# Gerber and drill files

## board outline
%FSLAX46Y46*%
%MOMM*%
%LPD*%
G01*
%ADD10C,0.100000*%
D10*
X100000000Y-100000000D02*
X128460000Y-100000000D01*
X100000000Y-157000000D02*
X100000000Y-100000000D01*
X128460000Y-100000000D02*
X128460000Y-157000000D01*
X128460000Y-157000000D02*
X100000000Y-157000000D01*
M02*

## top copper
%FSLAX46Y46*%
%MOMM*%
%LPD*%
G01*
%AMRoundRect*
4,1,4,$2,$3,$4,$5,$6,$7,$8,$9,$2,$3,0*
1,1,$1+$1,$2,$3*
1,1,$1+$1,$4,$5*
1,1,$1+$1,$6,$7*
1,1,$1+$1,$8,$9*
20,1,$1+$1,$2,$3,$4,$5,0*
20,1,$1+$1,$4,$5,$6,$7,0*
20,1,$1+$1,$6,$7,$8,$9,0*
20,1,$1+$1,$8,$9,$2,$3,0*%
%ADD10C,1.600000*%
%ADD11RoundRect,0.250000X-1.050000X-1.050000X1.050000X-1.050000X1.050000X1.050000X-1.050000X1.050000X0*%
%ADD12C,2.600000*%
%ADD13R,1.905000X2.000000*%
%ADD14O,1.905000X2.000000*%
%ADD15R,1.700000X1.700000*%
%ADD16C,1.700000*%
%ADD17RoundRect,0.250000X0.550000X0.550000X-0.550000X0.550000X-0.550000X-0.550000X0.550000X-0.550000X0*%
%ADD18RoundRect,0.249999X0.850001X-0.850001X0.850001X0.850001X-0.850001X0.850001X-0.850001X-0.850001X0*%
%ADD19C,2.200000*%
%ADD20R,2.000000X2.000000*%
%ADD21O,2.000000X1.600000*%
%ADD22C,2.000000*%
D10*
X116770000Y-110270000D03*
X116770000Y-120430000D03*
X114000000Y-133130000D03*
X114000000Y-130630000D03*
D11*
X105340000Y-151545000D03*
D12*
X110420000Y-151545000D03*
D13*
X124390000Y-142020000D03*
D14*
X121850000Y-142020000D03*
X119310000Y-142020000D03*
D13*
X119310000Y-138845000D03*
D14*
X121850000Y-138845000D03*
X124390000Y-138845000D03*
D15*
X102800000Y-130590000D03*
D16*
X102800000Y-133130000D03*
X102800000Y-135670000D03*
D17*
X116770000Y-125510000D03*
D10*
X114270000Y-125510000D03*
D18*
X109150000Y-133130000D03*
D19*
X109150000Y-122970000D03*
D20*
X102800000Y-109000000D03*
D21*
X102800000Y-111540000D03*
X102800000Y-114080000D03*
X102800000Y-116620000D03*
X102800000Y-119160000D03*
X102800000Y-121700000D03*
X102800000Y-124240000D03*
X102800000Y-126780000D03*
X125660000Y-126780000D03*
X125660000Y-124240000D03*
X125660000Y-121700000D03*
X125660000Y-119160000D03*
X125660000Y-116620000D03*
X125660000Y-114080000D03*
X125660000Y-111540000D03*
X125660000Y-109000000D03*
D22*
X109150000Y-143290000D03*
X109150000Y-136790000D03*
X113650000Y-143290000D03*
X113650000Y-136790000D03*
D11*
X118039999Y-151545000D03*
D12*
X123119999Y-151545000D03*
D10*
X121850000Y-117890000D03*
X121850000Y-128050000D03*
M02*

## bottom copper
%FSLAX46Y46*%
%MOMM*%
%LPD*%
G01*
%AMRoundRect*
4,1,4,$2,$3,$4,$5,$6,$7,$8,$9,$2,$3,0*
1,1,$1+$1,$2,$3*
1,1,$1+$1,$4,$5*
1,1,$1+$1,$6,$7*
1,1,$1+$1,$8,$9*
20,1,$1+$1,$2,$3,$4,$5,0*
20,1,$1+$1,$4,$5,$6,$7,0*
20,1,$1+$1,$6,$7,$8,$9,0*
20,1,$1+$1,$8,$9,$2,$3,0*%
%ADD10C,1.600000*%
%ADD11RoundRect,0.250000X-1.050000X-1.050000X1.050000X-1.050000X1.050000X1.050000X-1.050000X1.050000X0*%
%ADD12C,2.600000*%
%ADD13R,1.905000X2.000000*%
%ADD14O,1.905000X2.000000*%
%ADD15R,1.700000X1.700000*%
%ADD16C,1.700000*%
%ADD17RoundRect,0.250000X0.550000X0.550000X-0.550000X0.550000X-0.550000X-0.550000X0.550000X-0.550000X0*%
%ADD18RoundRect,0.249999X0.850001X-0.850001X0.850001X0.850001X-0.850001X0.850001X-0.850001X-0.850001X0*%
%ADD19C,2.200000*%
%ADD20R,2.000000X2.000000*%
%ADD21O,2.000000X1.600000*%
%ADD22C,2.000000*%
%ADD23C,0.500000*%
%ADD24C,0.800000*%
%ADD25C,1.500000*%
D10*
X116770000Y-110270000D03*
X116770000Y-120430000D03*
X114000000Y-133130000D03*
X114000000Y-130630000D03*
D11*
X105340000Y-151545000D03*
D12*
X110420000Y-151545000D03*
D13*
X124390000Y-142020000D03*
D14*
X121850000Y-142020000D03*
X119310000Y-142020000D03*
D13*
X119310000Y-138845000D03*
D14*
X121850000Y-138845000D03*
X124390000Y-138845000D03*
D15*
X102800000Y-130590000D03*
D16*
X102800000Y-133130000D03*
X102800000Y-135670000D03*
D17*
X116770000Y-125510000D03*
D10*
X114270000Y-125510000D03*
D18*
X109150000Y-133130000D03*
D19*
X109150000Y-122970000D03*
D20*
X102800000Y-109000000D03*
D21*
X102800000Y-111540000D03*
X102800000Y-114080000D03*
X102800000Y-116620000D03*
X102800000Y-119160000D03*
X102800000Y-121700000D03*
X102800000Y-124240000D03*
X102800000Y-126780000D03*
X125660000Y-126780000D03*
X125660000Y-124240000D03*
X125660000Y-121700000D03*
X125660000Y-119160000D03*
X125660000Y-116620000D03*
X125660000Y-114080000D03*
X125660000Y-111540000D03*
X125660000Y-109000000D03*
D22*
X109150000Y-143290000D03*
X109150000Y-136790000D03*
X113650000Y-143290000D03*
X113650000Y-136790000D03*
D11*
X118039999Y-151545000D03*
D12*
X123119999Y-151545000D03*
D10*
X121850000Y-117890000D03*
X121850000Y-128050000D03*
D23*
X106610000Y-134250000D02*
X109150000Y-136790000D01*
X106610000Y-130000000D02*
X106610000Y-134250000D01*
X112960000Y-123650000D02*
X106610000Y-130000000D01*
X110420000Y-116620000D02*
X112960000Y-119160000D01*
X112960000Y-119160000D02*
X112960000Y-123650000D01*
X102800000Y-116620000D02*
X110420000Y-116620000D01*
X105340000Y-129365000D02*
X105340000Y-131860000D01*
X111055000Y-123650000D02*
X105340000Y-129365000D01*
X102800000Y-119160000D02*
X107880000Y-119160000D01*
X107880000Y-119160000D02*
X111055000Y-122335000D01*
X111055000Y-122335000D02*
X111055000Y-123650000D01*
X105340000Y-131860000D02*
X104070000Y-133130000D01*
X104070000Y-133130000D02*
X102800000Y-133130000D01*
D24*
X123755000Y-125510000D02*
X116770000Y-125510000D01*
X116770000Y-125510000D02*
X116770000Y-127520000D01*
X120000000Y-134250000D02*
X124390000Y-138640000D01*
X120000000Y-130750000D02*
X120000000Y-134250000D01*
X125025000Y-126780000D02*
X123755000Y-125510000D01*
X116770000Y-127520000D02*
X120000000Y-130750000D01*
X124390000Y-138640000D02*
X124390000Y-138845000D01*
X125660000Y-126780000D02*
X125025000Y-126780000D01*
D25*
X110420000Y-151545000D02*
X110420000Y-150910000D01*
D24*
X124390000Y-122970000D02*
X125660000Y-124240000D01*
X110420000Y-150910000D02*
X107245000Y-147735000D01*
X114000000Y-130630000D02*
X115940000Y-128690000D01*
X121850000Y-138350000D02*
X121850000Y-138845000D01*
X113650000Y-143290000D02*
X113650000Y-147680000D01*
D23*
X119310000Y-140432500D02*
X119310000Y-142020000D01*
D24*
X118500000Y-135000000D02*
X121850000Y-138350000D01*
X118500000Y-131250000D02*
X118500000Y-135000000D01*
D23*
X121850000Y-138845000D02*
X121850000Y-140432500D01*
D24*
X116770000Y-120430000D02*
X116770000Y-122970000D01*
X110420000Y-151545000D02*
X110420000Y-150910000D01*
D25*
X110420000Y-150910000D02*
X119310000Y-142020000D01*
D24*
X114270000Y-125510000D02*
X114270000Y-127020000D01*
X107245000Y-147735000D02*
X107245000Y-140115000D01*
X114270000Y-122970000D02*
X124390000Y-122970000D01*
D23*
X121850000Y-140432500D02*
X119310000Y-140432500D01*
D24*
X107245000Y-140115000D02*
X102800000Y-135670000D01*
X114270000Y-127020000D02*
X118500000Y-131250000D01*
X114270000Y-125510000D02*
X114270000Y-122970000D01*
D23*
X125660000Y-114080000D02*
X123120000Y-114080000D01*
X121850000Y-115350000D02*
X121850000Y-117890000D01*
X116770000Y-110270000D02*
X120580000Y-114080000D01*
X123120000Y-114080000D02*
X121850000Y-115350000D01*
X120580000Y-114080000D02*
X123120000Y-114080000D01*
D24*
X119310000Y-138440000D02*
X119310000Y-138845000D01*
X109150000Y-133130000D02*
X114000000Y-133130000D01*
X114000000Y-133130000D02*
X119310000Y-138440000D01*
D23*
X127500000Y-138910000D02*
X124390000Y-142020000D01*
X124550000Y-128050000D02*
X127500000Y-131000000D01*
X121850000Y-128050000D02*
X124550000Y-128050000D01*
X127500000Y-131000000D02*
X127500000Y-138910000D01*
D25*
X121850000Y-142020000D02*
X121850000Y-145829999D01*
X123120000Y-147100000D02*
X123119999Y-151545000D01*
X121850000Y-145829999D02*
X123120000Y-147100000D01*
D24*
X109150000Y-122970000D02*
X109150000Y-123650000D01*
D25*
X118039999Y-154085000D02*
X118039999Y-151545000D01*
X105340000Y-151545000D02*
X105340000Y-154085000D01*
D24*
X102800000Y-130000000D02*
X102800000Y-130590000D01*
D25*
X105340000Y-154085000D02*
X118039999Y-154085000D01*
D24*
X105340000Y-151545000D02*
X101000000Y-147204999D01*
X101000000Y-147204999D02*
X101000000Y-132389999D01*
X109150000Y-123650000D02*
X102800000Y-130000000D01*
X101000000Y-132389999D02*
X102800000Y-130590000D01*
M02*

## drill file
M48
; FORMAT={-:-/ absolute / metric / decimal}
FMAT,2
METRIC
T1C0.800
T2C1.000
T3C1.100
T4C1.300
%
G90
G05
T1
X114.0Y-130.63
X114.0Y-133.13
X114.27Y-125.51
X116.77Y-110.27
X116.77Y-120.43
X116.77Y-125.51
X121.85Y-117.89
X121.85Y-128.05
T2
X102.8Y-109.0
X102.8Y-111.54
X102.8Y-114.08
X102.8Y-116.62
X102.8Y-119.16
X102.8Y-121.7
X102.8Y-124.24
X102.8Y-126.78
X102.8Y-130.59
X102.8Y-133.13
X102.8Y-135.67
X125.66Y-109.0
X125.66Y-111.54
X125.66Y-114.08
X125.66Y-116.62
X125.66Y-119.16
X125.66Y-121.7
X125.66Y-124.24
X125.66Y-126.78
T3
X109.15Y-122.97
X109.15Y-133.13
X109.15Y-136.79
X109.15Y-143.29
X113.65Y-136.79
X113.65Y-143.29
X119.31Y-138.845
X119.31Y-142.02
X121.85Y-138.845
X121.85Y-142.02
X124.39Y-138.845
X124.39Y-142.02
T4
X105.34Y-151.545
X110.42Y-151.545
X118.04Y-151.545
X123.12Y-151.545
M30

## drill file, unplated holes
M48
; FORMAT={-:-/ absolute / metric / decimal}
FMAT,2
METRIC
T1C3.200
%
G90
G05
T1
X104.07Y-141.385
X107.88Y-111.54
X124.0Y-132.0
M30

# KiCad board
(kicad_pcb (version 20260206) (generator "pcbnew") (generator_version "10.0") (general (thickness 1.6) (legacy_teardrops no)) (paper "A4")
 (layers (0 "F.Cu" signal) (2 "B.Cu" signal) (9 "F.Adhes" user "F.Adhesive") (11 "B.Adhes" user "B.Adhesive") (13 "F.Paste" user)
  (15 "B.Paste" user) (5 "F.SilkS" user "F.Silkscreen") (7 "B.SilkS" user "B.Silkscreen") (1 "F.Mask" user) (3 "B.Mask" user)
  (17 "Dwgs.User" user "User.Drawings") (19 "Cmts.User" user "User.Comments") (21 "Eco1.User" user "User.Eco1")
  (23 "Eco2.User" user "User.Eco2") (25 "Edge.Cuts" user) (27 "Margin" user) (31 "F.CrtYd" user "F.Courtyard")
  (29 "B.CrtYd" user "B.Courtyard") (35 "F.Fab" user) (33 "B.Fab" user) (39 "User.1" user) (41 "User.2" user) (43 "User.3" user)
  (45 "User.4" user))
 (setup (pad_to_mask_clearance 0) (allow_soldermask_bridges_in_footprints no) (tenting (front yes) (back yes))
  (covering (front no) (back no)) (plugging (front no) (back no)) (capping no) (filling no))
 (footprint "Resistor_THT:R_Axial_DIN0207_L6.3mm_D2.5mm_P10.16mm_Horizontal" (layer "F.Cu") (at 116.77 110.27 -90)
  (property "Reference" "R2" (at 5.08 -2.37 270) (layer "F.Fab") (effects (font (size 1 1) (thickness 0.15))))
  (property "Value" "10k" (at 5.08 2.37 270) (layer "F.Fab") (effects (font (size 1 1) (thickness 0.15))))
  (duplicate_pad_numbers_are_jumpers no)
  (pad "1" thru_hole circle (at 0 0 270) (size 1.6 1.6) (drill 0.8) (layers "*.Cu" "*.Mask") (remove_unused_layers no) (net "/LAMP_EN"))
  (pad "2" thru_hole circle (at 10.16 0 270) (size 1.6 1.6) (drill 0.8) (layers "*.Cu" "*.Mask") (remove_unused_layers no) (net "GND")))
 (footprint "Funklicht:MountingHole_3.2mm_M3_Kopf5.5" (layer "F.Cu") (at 107.88 111.539999)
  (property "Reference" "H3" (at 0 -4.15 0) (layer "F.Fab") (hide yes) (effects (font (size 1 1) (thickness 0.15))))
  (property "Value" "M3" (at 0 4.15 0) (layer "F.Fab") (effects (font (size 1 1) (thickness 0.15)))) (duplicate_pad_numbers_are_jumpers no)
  (pad "" np_thru_hole circle (at 0 0) (size 3.2 3.2) (drill 3.2) (layers "*.Cu" "*.Mask")))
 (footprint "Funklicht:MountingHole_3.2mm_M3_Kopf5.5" (layer "F.Cu") (at 104.07 141.385)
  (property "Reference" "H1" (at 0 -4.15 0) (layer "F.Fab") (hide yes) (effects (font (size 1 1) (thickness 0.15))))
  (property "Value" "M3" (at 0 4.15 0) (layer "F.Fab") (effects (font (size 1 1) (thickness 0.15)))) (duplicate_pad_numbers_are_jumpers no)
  (pad "" np_thru_hole circle (at 0 0) (size 3.2 3.2) (drill 3.2) (layers "*.Cu" "*.Mask")))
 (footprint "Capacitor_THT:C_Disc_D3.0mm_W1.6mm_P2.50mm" (layer "F.Cu") (at 114 133.13 90)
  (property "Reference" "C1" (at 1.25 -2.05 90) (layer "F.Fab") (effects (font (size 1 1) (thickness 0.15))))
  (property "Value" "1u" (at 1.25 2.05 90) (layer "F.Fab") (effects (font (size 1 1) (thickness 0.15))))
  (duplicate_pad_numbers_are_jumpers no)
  (pad "1" thru_hole circle (at 0 0 90) (size 1.6 1.6) (drill 0.8) (layers "*.Cu" "*.Mask") (remove_unused_layers no) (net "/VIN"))
  (pad "2" thru_hole circle (at 2.5 0 90) (size 1.6 1.6) (drill 0.8) (layers "*.Cu" "*.Mask") (remove_unused_layers no) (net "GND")))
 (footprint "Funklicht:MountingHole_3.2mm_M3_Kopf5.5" (layer "F.Cu") (at 124 132)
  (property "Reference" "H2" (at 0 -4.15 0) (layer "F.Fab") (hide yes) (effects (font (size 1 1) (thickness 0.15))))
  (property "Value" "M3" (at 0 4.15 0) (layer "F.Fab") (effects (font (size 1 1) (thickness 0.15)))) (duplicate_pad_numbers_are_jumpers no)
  (pad "" np_thru_hole circle (at 0 0) (size 3.2 3.2) (drill 3.2) (layers "*.Cu" "*.Mask")))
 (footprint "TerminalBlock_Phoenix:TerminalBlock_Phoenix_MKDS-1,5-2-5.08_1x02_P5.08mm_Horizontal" (layer "F.Cu") (at 105.34 151.545)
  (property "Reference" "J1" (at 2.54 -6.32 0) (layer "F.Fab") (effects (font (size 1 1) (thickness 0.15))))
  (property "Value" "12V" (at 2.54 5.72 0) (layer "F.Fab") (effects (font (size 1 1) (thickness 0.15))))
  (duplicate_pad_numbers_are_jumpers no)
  (pad "1" thru_hole roundrect (at 0 0) (size 2.6 2.6) (drill 1.3) (layers "*.Cu" "*.Mask") (remove_unused_layers no)
   (roundrect_rratio 0.096154) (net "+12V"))
  (pad "2" thru_hole circle (at 5.08 0) (size 2.6 2.6) (drill 1.3) (layers "*.Cu" "*.Mask") (remove_unused_layers no) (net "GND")))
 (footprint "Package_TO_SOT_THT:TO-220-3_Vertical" (layer "F.Cu") (at 124.39 142.02 180)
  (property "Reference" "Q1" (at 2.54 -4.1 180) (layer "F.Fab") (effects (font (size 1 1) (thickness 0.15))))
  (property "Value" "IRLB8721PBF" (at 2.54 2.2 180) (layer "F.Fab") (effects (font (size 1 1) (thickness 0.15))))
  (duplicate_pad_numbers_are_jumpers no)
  (pad "1" thru_hole rect (at 0 0 180) (size 1.905 2) (drill 1.1) (layers "*.Cu" "*.Mask") (remove_unused_layers no) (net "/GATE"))
  (pad "2" thru_hole oval (at 2.54 0 180) (size 1.905 2) (drill 1.1) (layers "*.Cu" "*.Mask") (remove_unused_layers no) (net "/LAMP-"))
  (pad "3" thru_hole oval (at 5.08 0 180) (size 1.905 2) (drill 1.1) (layers "*.Cu" "*.Mask") (remove_unused_layers no) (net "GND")))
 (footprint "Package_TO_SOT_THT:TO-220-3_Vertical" (layer "F.Cu") (at 119.31 138.845)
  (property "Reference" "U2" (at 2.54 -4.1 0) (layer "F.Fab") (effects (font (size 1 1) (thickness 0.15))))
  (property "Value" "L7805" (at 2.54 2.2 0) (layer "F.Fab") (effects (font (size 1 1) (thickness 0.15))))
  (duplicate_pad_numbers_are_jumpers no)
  (pad "1" thru_hole rect (at 0 0) (size 1.905 2) (drill 1.1) (layers "*.Cu" "*.Mask") (remove_unused_layers no) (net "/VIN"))
  (pad "2" thru_hole oval (at 2.54 0) (size 1.905 2) (drill 1.1) (layers "*.Cu" "*.Mask") (remove_unused_layers no) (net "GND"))
  (pad "3" thru_hole oval (at 5.08 0) (size 1.905 2) (drill 1.1) (layers "*.Cu" "*.Mask") (remove_unused_layers no) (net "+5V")))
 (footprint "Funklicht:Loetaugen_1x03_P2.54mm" (layer "F.Cu") (at 102.8 130.59)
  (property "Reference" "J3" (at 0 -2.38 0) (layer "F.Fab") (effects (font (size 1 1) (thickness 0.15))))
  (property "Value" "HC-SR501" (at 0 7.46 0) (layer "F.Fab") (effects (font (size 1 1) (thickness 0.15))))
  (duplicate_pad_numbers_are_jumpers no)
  (pad "1" thru_hole rect (at 0 0) (size 1.7 1.7) (drill 1) (layers "*.Cu" "*.Mask") (remove_unused_layers no) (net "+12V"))
  (pad "2" thru_hole circle (at 0 2.54) (size 1.7 1.7) (drill 1) (layers "*.Cu" "*.Mask") (remove_unused_layers no) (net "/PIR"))
  (pad "3" thru_hole circle (at 0 5.08) (size 1.7 1.7) (drill 1) (layers "*.Cu" "*.Mask") (remove_unused_layers no) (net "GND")))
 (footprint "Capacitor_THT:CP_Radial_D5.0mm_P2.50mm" (layer "F.Cu") (at 116.77 125.51 180)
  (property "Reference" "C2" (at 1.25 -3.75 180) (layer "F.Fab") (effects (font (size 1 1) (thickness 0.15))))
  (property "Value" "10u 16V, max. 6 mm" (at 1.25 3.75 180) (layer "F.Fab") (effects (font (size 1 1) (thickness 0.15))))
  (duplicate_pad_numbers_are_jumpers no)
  (pad "1" thru_hole roundrect (at 0 0 180) (size 1.6 1.6) (drill 0.8) (layers "*.Cu" "*.Mask") (remove_unused_layers no)
   (roundrect_rratio 0.15625) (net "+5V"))
  (pad "2" thru_hole circle (at 2.5 0 180) (size 1.6 1.6) (drill 0.8) (layers "*.Cu" "*.Mask") (remove_unused_layers no) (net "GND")))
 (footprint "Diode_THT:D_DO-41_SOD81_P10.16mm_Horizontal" (layer "F.Cu") (at 109.15 133.13 90)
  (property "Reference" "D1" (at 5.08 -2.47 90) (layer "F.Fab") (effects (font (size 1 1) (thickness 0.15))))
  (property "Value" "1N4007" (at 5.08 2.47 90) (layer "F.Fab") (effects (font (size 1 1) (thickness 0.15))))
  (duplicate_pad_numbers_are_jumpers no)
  (pad "1" thru_hole roundrect (at 0 0 90) (size 2.2 2.2) (drill 1.1) (layers "*.Cu" "*.Mask") (remove_unused_layers no)
   (roundrect_rratio 0.113636) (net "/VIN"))
  (pad "2" thru_hole circle (at 10.16 0 90) (size 2.2 2.2) (drill 1.1) (layers "*.Cu" "*.Mask") (remove_unused_layers no) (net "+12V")))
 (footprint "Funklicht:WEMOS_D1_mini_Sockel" (layer "F.Cu") (at 102.8 109)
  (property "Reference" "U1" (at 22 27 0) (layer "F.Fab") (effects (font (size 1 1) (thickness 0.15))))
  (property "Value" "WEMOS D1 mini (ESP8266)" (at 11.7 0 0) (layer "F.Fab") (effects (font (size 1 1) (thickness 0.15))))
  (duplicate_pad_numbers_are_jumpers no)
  (pad "1" thru_hole rect (at 0 0) (size 2 2) (drill 1) (layers "*.Cu" "*.Mask") (remove_unused_layers no)
   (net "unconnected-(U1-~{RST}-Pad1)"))
  (pad "2" thru_hole oval (at 0 2.54) (size 2 1.6) (drill 1) (layers "*.Cu" "*.Mask") (remove_unused_layers no)
   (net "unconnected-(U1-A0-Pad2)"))
  (pad "3" thru_hole oval (at 0 5.08) (size 2 1.6) (drill 1) (layers "*.Cu" "*.Mask") (remove_unused_layers no)
   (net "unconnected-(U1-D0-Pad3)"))
  (pad "4" thru_hole oval (at 0 7.62) (size 2 1.6) (drill 1) (layers "*.Cu" "*.Mask") (remove_unused_layers no) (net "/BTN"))
  (pad "5" thru_hole oval (at 0 10.16) (size 2 1.6) (drill 1) (layers "*.Cu" "*.Mask") (remove_unused_layers no) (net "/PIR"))
  (pad "6" thru_hole oval (at 0 12.7) (size 2 1.6) (drill 1) (layers "*.Cu" "*.Mask") (remove_unused_layers no)
   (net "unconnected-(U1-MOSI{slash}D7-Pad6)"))
  (pad "7" thru_hole oval (at 0 15.24) (size 2 1.6) (drill 1) (layers "*.Cu" "*.Mask") (remove_unused_layers no)
   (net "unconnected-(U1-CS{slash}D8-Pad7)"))
  (pad "8" thru_hole oval (at 0 17.78) (size 2 1.6) (drill 1) (layers "*.Cu" "*.Mask") (remove_unused_layers no)
   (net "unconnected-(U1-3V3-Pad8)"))
  (pad "9" thru_hole oval (at 22.86 17.78) (size 2 1.6) (drill 1) (layers "*.Cu" "*.Mask") (remove_unused_layers no) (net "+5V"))
  (pad "10" thru_hole oval (at 22.86 15.24) (size 2 1.6) (drill 1) (layers "*.Cu" "*.Mask") (remove_unused_layers no) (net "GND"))
  (pad "11" thru_hole oval (at 22.86 12.7) (size 2 1.6) (drill 1) (layers "*.Cu" "*.Mask") (remove_unused_layers no)
   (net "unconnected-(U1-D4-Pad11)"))
  (pad "12" thru_hole oval (at 22.86 10.16) (size 2 1.6) (drill 1) (layers "*.Cu" "*.Mask") (remove_unused_layers no)
   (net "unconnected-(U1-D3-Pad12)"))
  (pad "13" thru_hole oval (at 22.86 7.62) (size 2 1.6) (drill 1) (layers "*.Cu" "*.Mask") (remove_unused_layers no)
   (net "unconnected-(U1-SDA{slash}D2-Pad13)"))
  (pad "14" thru_hole oval (at 22.86 5.08) (size 2 1.6) (drill 1) (layers "*.Cu" "*.Mask") (remove_unused_layers no) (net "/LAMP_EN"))
  (pad "15" thru_hole oval (at 22.86 2.54) (size 2 1.6) (drill 1) (layers "*.Cu" "*.Mask") (remove_unused_layers no)
   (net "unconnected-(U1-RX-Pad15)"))
  (pad "16" thru_hole oval (at 22.86 0) (size 2 1.6) (drill 1) (layers "*.Cu" "*.Mask") (remove_unused_layers no)
   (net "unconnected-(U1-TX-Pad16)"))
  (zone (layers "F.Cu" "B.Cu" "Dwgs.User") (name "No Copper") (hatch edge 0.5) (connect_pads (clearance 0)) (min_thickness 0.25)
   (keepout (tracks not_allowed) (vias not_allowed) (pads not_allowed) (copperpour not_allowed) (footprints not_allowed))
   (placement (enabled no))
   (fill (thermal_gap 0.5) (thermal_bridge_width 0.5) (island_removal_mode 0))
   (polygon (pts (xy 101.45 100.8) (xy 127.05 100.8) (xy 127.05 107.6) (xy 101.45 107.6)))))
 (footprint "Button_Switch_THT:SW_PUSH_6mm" (layer "F.Cu") (at 109.15 143.29 90)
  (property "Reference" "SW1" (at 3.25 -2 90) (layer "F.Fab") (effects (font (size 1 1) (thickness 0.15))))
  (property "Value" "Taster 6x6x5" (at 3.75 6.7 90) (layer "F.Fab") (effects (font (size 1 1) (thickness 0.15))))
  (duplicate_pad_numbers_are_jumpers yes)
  (pad "1" thru_hole circle (at 0 0 180) (size 2 2) (drill 1.1) (layers "*.Cu" "*.Mask") (remove_unused_layers no) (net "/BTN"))
  (pad "1" thru_hole circle (at 6.5 0 180) (size 2 2) (drill 1.1) (layers "*.Cu" "*.Mask") (remove_unused_layers no) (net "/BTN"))
  (pad "2" thru_hole circle (at 0 4.5 180) (size 2 2) (drill 1.1) (layers "*.Cu" "*.Mask") (remove_unused_layers no) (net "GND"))
  (pad "2" thru_hole circle (at 6.5 4.5 180) (size 2 2) (drill 1.1) (layers "*.Cu" "*.Mask") (remove_unused_layers no) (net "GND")))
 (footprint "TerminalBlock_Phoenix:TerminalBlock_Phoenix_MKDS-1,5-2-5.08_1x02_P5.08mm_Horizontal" (layer "F.Cu") (at 118.039999 151.545)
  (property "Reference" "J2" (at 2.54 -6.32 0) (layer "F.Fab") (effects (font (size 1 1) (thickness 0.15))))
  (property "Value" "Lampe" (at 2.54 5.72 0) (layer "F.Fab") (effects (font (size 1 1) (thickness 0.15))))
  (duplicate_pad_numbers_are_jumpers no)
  (pad "1" thru_hole roundrect (at 0 0) (size 2.6 2.6) (drill 1.3) (layers "*.Cu" "*.Mask") (remove_unused_layers no)
   (roundrect_rratio 0.096154) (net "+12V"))
  (pad "2" thru_hole circle (at 5.08 0) (size 2.6 2.6) (drill 1.3) (layers "*.Cu" "*.Mask") (remove_unused_layers no) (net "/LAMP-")))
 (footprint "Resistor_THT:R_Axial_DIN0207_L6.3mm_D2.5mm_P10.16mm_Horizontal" (layer "F.Cu") (at 121.85 117.89 -90)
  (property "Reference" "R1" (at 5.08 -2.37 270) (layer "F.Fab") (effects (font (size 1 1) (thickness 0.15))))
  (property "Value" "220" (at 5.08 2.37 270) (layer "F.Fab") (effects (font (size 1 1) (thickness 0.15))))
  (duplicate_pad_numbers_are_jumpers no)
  (pad "1" thru_hole circle (at 0 0 270) (size 1.6 1.6) (drill 0.8) (layers "*.Cu" "*.Mask") (remove_unused_layers no) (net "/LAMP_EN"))
  (pad "2" thru_hole circle (at 10.16 0 270) (size 1.6 1.6) (drill 0.8) (layers "*.Cu" "*.Mask") (remove_unused_layers no) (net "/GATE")))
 (gr_line (start 100 100) (end 128.46 100) (stroke (width 0.1) (type default)) (layer "Edge.Cuts"))
 (gr_line (start 100 157) (end 100 100) (stroke (width 0.1) (type default)) (layer "Edge.Cuts"))
 (gr_line (start 128.46 100) (end 128.46 157) (stroke (width 0.1) (type default)) (layer "Edge.Cuts"))
 (gr_line (start 128.46 157) (end 100 157) (stroke (width 0.1) (type default)) (layer "Edge.Cuts"))
 (segment (start 106.61 134.25) (end 109.15 136.79) (width 0.5) (layer "B.Cu") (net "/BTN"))
 (segment (start 106.61 130) (end 106.61 134.25) (width 0.5) (layer "B.Cu") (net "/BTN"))
 (segment (start 112.96 123.65) (end 106.61 130) (width 0.5) (layer "B.Cu") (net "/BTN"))
 (segment (start 110.42 116.62) (end 112.96 119.16) (width 0.5) (layer "B.Cu") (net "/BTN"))
 (segment (start 112.96 119.16) (end 112.96 123.65) (width 0.5) (layer "B.Cu") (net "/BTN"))
 (segment (start 102.8 116.62) (end 110.42 116.62) (width 0.5) (layer "B.Cu") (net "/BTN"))
 (segment (start 105.34 129.365) (end 105.34 131.86) (width 0.5) (layer "B.Cu") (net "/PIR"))
 (segment (start 111.055 123.65) (end 105.34 129.365) (width 0.5) (layer "B.Cu") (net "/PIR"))
 (segment (start 102.8 119.16) (end 107.88 119.16) (width 0.5) (layer "B.Cu") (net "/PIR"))
 (segment (start 107.88 119.16) (end 111.055 122.335) (width 0.5) (layer "B.Cu") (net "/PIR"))
 (segment (start 111.055 122.335) (end 111.055 123.65) (width 0.5) (layer "B.Cu") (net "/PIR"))
 (segment (start 105.34 131.86) (end 104.07 133.13) (width 0.5) (layer "B.Cu") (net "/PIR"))
 (segment (start 104.07 133.13) (end 102.8 133.13) (width 0.5) (layer "B.Cu") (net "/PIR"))
 (segment (start 123.755 125.51) (end 116.77 125.51) (width 0.8) (layer "B.Cu") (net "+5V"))
 (segment (start 116.77 125.51) (end 116.77 127.52) (width 0.8) (layer "B.Cu") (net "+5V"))
 (segment (start 120 134.25) (end 124.39 138.64) (width 0.8) (layer "B.Cu") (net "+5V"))
 (segment (start 120 130.75) (end 120 134.25) (width 0.8) (layer "B.Cu") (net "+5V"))
 (segment (start 125.025 126.78) (end 123.755 125.51) (width 0.8) (layer "B.Cu") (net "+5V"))
 (segment (start 116.77 127.52) (end 120 130.75) (width 0.8) (layer "B.Cu") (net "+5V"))
 (segment (start 124.39 138.64) (end 124.39 138.845) (width 0.8) (layer "B.Cu") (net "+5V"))
 (segment (start 125.66 126.78) (end 125.025 126.78) (width 0.8) (layer "B.Cu") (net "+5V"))
 (segment (start 110.42 151.545) (end 110.42 150.91) (width 1.5) (layer "B.Cu") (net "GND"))
 (segment (start 124.39 122.97) (end 125.66 124.24) (width 0.8) (layer "B.Cu") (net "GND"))
 (segment (start 110.42 150.91) (end 107.245 147.735) (width 0.8) (layer "B.Cu") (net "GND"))
 (segment (start 114 130.63) (end 115.94 128.69) (width 0.8) (layer "B.Cu") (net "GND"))
 (segment (start 121.85 138.35) (end 121.85 138.845) (width 0.8) (layer "B.Cu") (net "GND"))
 (segment (start 113.65 143.29) (end 113.65 147.68) (width 0.8) (layer "B.Cu") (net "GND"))
 (segment (start 119.31 140.4325) (end 119.31 142.02) (width 0.5) (layer "B.Cu") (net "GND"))
 (segment (start 118.5 135) (end 121.85 138.35) (width 0.8) (layer "B.Cu") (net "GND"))
 (segment (start 118.5 131.25) (end 118.5 135) (width 0.8) (layer "B.Cu") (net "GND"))
 (segment (start 121.85 138.845) (end 121.85 140.4325) (width 0.5) (layer "B.Cu") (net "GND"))
 (segment (start 116.77 120.43) (end 116.77 122.97) (width 0.8) (layer "B.Cu") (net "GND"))
 (segment (start 110.42 151.545) (end 110.42 150.91) (width 0.8) (layer "B.Cu") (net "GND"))
 (segment (start 110.42 150.91) (end 119.31 142.02) (width 1.5) (layer "B.Cu") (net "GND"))
 (segment (start 114.27 125.51) (end 114.27 127.02) (width 0.8) (layer "B.Cu") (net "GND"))
 (segment (start 107.245 147.735) (end 107.245 140.115) (width 0.8) (layer "B.Cu") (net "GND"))
 (segment (start 114.27 122.97) (end 124.39 122.97) (width 0.8) (layer "B.Cu") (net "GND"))
 (segment (start 121.85 140.4325) (end 119.31 140.4325) (width 0.5) (layer "B.Cu") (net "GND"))
 (segment (start 107.245 140.115) (end 102.8 135.67) (width 0.8) (layer "B.Cu") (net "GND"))
 (segment (start 114.27 127.02) (end 118.5 131.25) (width 0.8) (layer "B.Cu") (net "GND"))
 (segment (start 114.27 125.51) (end 114.27 122.97) (width 0.8) (layer "B.Cu") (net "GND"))
 (segment (start 125.66 114.08) (end 123.12 114.08) (width 0.5) (layer "B.Cu") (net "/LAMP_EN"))
 (segment (start 121.85 115.35) (end 121.85 117.89) (width 0.5) (layer "B.Cu") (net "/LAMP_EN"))
 (segment (start 116.77 110.27) (end 120.58 114.08) (width 0.5) (layer "B.Cu") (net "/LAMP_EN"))
 (segment (start 123.12 114.08) (end 121.85 115.35) (width 0.5) (layer "B.Cu") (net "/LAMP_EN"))
 (segment (start 120.58 114.08) (end 123.12 114.08) (width 0.5) (layer "B.Cu") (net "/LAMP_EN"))
 (segment (start 119.31 138.44) (end 119.31 138.845) (width 0.8) (layer "B.Cu") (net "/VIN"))
 (segment (start 109.15 133.13) (end 114 133.13) (width 0.8) (layer "B.Cu") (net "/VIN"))
 (segment (start 114 133.13) (end 119.31 138.44) (width 0.8) (layer "B.Cu") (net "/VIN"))
 (segment (start 127.5 138.91) (end 124.39 142.02) (width 0.5) (layer "B.Cu") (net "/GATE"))
 (segment (start 124.55 128.05) (end 127.5 131) (width 0.5) (layer "B.Cu") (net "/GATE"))
 (segment (start 121.85 128.05) (end 124.55 128.05) (width 0.5) (layer "B.Cu") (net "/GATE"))
 (segment (start 127.5 131) (end 127.5 138.91) (width 0.5) (layer "B.Cu") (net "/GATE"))
 (segment (start 121.85 142.02) (end 121.85 145.829999) (width 1.5) (layer "B.Cu") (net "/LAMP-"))
 (segment (start 123.12 147.1) (end 123.119999 151.545) (width 1.5) (layer "B.Cu") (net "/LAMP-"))
 (segment (start 121.85 145.829999) (end 123.12 147.1) (width 1.5) (layer "B.Cu") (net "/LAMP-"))
 (segment (start 109.15 122.97) (end 109.15 123.65) (width 0.8) (layer "B.Cu") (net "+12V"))
 (segment (start 118.039999 154.085) (end 118.039999 151.545) (width 1.5) (layer "B.Cu") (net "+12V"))
 (segment (start 105.34 151.545) (end 105.34 154.085) (width 1.5) (layer "B.Cu") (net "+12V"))
 (segment (start 102.8 130) (end 102.8 130.59) (width 0.8) (layer "B.Cu") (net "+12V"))
 (segment (start 105.34 154.085) (end 118.039999 154.085) (width 1.5) (layer "B.Cu") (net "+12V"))
 (segment (start 105.34 151.545) (end 101 147.204999) (width 0.8) (layer "B.Cu") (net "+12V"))
 (segment (start 101 147.204999) (end 101 132.389999) (width 0.8) (layer "B.Cu") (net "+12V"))
 (segment (start 109.15 123.65) (end 102.8 130) (width 0.8) (layer "B.Cu") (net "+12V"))
 (segment (start 101 132.389999) (end 102.8 130.59) (width 0.8) (layer "B.Cu") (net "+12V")))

